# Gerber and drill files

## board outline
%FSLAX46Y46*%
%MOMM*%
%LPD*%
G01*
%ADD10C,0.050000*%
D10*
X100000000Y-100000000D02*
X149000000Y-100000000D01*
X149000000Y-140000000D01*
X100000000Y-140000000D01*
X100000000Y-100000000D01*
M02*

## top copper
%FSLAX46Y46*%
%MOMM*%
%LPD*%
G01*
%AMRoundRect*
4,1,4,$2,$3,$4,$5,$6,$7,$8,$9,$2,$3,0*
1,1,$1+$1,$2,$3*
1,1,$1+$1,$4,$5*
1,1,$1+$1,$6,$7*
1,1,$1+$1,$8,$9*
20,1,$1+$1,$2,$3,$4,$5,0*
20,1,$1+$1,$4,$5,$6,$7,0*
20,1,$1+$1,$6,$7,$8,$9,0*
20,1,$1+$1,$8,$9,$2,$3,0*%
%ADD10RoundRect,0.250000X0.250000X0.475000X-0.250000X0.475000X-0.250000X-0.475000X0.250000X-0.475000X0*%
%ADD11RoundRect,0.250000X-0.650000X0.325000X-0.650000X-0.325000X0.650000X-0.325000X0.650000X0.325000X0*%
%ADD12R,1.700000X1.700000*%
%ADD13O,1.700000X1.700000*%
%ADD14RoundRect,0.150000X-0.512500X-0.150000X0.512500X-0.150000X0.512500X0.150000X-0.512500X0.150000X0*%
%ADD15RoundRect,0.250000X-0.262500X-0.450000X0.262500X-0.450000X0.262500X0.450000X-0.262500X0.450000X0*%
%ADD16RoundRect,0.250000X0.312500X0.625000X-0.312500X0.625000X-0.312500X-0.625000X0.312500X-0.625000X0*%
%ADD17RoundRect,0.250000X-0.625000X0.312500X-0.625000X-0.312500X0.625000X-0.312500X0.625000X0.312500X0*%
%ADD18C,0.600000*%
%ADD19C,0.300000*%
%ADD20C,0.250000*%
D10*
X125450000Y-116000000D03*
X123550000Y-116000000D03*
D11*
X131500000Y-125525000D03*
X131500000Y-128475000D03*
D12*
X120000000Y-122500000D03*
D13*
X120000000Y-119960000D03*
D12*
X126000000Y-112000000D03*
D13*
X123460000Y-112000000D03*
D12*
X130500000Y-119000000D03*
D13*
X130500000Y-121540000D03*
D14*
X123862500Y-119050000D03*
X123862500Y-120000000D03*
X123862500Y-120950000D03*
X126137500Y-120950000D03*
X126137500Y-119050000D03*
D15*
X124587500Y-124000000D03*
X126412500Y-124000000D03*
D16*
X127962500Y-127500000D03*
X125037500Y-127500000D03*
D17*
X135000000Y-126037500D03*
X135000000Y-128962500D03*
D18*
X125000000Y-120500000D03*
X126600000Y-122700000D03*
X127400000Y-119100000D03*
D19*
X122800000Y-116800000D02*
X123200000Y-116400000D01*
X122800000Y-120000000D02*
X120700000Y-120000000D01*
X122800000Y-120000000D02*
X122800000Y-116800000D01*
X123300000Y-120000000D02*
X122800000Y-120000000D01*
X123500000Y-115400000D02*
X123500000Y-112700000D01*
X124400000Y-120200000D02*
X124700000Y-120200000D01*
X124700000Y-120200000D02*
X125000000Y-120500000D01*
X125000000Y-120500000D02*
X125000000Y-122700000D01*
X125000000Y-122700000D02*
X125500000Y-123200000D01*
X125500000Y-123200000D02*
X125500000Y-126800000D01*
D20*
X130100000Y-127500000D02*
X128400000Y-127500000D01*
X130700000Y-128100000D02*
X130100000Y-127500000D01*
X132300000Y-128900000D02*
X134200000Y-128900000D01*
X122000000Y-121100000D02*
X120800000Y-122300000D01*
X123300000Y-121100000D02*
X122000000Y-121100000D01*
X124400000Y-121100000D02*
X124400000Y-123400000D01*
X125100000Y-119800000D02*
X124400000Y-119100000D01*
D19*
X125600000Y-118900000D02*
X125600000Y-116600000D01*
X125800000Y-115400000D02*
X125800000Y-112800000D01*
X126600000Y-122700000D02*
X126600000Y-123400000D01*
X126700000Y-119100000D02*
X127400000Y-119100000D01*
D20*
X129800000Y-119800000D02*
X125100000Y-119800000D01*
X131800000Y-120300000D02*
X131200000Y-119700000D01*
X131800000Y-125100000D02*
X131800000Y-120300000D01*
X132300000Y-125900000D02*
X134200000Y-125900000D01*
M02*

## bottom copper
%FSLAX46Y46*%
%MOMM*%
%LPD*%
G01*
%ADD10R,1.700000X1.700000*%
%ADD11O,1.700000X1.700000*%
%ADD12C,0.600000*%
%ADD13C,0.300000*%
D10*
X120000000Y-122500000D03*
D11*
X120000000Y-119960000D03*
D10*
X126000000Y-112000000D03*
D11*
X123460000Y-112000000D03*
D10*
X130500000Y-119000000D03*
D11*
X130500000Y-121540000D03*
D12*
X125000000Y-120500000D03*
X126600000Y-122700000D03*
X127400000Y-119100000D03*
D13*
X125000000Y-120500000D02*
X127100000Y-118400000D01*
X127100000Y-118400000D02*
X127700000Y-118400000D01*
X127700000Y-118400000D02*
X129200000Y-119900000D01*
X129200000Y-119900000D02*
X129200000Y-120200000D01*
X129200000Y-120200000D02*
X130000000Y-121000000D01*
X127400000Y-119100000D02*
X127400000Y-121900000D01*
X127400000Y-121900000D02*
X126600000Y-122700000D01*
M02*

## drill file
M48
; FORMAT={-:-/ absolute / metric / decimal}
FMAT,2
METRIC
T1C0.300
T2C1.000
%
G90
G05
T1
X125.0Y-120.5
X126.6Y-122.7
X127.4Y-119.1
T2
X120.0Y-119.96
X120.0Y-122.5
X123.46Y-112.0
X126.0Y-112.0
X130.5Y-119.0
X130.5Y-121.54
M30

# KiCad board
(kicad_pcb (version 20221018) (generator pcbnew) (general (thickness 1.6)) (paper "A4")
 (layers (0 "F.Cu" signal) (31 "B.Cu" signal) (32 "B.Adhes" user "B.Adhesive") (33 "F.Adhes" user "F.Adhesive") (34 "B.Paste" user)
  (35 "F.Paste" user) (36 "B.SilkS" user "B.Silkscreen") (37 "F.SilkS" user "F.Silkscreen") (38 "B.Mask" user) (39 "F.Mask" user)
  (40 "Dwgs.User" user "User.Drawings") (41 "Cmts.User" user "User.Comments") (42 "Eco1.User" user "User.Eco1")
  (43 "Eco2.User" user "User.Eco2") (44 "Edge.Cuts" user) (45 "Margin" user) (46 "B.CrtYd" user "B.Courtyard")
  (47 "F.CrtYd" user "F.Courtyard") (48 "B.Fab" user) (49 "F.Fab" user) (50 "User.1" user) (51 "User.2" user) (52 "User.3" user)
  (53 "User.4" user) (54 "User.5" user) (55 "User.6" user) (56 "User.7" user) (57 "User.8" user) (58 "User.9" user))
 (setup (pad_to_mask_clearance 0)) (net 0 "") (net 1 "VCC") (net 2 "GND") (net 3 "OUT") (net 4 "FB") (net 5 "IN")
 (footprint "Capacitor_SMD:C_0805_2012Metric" (layer "F.Cu") (at 124.5 116 180)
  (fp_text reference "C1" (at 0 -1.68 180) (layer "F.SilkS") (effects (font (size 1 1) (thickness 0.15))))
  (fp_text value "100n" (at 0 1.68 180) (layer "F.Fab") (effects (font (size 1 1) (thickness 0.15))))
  (pad "1" smd roundrect (at -0.95 0 180) (size 1 1.45) (layers "F.Cu" "F.Paste" "F.Mask") (roundrect_rratio 0.25) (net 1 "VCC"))
  (pad "2" smd roundrect (at 0.95 0 180) (size 1 1.45) (layers "F.Cu" "F.Paste" "F.Mask") (roundrect_rratio 0.25) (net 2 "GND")))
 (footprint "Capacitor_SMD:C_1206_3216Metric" (layer "F.Cu") (at 131.5 127 -90)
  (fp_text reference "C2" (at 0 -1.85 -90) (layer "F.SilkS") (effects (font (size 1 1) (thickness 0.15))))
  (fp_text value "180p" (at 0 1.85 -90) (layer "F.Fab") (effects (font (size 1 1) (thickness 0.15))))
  (pad "1" smd roundrect (at -1.475 0 270) (size 1.15 1.8) (layers "F.Cu" "F.Paste" "F.Mask") (roundrect_rratio 0.217391) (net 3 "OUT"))
  (pad "2" smd roundrect (at 1.475 0 270) (size 1.15 1.8) (layers "F.Cu" "F.Paste" "F.Mask") (roundrect_rratio 0.217391) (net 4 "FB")))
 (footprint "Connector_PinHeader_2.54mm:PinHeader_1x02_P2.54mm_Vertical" (layer "F.Cu") (at 120 122.5 180)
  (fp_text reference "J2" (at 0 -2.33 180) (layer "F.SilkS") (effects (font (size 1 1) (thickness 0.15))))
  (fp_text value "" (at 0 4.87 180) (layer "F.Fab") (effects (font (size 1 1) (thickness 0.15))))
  (pad "1" thru_hole rect (at 0 0 180) (size 1.7 1.7) (drill 1) (layers "*.Cu" "*.Mask") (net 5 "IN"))
  (pad "2" thru_hole oval (at 0 2.54 180) (size 1.7 1.7) (drill 1) (layers "*.Cu" "*.Mask") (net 2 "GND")))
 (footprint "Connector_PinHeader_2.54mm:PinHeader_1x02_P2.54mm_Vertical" (layer "F.Cu") (at 126 112 -90)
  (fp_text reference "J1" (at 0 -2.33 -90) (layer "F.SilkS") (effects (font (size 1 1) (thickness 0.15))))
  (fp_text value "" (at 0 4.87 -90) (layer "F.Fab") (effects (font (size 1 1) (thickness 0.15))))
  (pad "1" thru_hole rect (at 0 0 270) (size 1.7 1.7) (drill 1) (layers "*.Cu" "*.Mask") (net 1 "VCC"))
  (pad "2" thru_hole oval (at 0 2.54 270) (size 1.7 1.7) (drill 1) (layers "*.Cu" "*.Mask") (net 2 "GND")))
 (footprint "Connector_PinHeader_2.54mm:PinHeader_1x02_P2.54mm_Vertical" (layer "F.Cu") (at 130.5 119)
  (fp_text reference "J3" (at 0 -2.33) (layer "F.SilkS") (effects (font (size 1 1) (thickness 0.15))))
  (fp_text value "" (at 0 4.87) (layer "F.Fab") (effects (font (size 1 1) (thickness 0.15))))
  (pad "1" thru_hole rect (at 0 0) (size 1.7 1.7) (drill 1) (layers "*.Cu" "*.Mask") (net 3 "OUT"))
  (pad "2" thru_hole oval (at 0 2.54) (size 1.7 1.7) (drill 1) (layers "*.Cu" "*.Mask") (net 2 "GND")))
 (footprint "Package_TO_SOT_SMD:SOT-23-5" (layer "F.Cu") (at 125 120)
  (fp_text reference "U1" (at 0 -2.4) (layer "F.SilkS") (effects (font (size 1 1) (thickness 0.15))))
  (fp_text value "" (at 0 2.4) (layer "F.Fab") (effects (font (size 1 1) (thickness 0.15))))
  (pad "1" smd roundrect (at -1.1375 -0.95) (size 1.325 0.6) (layers "F.Cu" "F.Paste" "F.Mask") (roundrect_rratio 0.25) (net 3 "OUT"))
  (pad "2" smd roundrect (at -1.1375 0) (size 1.325 0.6) (layers "F.Cu" "F.Paste" "F.Mask") (roundrect_rratio 0.25) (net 2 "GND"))
  (pad "3" smd roundrect (at -1.1375 0.95) (size 1.325 0.6) (layers "F.Cu" "F.Paste" "F.Mask") (roundrect_rratio 0.25) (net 5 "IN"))
  (pad "4" smd roundrect (at 1.1375 0.95) (size 1.325 0.6) (layers "F.Cu" "F.Paste" "F.Mask") (roundrect_rratio 0.25))
  (pad "5" smd roundrect (at 1.1375 -0.95) (size 1.325 0.6) (layers "F.Cu" "F.Paste" "F.Mask") (roundrect_rratio 0.25) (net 1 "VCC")))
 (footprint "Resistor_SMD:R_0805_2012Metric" (layer "F.Cu") (at 125.5 124)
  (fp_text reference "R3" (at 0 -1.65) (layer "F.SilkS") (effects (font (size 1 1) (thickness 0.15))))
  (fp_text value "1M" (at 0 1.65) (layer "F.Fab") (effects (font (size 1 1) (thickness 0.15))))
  (pad "1" smd roundrect (at -0.9125 0) (size 1.025 1.4) (layers "F.Cu" "F.Paste" "F.Mask") (roundrect_rratio 0.243902) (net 5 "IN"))
  (pad "2" smd roundrect (at 0.9125 0) (size 1.025 1.4) (layers "F.Cu" "F.Paste" "F.Mask") (roundrect_rratio 0.243902) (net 1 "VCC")))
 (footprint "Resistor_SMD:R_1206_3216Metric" (layer "F.Cu") (at 126.5 127.5 180)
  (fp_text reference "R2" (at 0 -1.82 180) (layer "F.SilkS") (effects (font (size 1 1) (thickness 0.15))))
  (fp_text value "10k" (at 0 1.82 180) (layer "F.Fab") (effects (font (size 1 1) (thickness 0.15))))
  (pad "1" smd roundrect (at -1.4625 0 180) (size 1.125 1.75) (layers "F.Cu" "F.Paste" "F.Mask") (roundrect_rratio 0.222222) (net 4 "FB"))
  (pad "2" smd roundrect (at 1.4625 0 180) (size 1.125 1.75) (layers "F.Cu" "F.Paste" "F.Mask") (roundrect_rratio 0.222222) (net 2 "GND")))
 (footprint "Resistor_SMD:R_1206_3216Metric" (layer "F.Cu") (at 135 127.5 -90)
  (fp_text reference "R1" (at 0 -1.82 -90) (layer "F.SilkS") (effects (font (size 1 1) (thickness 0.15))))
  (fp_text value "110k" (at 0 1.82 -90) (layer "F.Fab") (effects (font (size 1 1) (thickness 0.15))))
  (pad "1" smd roundrect (at -1.4625 0 270) (size 1.125 1.75) (layers "F.Cu" "F.Paste" "F.Mask") (roundrect_rratio 0.222222) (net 3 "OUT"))
  (pad "2" smd roundrect (at 1.4625 0 270) (size 1.125 1.75) (layers "F.Cu" "F.Paste" "F.Mask") (roundrect_rratio 0.222222) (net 4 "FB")))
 (gr_rect (start 100 100) (end 149 140) (stroke (width 0.05) (type default)) (fill none) (layer "Edge.Cuts"))
 (segment (start 122.8 116.8) (end 123.2 116.4) (width 0.3) (layer "F.Cu") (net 2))
 (segment (start 122.8 120) (end 120.7 120) (width 0.3) (layer "F.Cu") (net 2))
 (segment (start 122.8 120) (end 122.8 116.8) (width 0.3) (layer "F.Cu") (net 2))
 (segment (start 123.3 120) (end 122.8 120) (width 0.3) (layer "F.Cu") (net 2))
 (segment (start 123.5 115.4) (end 123.5 112.7) (width 0.3) (layer "F.Cu") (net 2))
 (segment (start 124.4 120.2) (end 124.7 120.2) (width 0.3) (layer "F.Cu") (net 2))
 (segment (start 124.7 120.2) (end 125 120.5) (width 0.3) (layer "F.Cu") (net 2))
 (segment (start 125 120.5) (end 125 122.7) (width 0.3) (layer "F.Cu") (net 2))
 (segment (start 125 122.7) (end 125.5 123.2) (width 0.3) (layer "F.Cu") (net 2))
 (segment (start 125.5 123.2) (end 125.5 126.8) (width 0.3) (layer "F.Cu") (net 2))
 (segment (start 130.1 127.5) (end 128.4 127.5) (width 0.25) (layer "F.Cu") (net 4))
 (segment (start 130.7 128.1) (end 130.1 127.5) (width 0.25) (layer "F.Cu") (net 4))
 (segment (start 132.3 128.9) (end 134.2 128.9) (width 0.25) (layer "F.Cu") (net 4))
 (via (at 125 120.5) (size 0.6) (drill 0.3) (layers "F.Cu" "B.Cu") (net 2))
 (segment (start 122 121.1) (end 120.8 122.3) (width 0.25) (layer "F.Cu") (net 5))
 (segment (start 123.3 121.1) (end 122 121.1) (width 0.25) (layer "F.Cu") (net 5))
 (segment (start 124.4 121.1) (end 124.4 123.4) (width 0.25) (layer "F.Cu") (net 5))
 (segment (start 125 120.5) (end 127.1 118.4) (width 0.3) (layer "B.Cu") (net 2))
 (segment (start 125.1 119.8) (end 124.4 119.1) (width 0.25) (layer "F.Cu") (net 3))
 (segment (start 125.6 118.9) (end 125.6 116.6) (width 0.3) (layer "F.Cu") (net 1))
 (segment (start 125.8 115.4) (end 125.8 112.8) (width 0.3) (layer "F.Cu") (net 1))
 (segment (start 126.6 122.7) (end 126.6 123.4) (width 0.3) (layer "F.Cu") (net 1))
 (segment (start 126.7 119.1) (end 127.4 119.1) (width 0.3) (layer "F.Cu") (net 1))
 (segment (start 127.1 118.4) (end 127.7 118.4) (width 0.3) (layer "B.Cu") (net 2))
 (segment (start 127.7 118.4) (end 129.2 119.9) (width 0.3) (layer "B.Cu") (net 2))
 (segment (start 129.2 119.9) (end 129.2 120.2) (width 0.3) (layer "B.Cu") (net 2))
 (segment (start 129.2 120.2) (end 130 121) (width 0.3) (layer "B.Cu") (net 2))
 (segment (start 129.8 119.8) (end 125.1 119.8) (width 0.25) (layer "F.Cu") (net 3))
 (segment (start 131.8 120.3) (end 131.2 119.7) (width 0.25) (layer "F.Cu") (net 3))
 (segment (start 131.8 125.1) (end 131.8 120.3) (width 0.25) (layer "F.Cu") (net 3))
 (segment (start 132.3 125.9) (end 134.2 125.9) (width 0.25) (layer "F.Cu") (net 3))
 (via (at 126.6 122.7) (size 0.6) (drill 0.3) (layers "F.Cu" "B.Cu") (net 1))
 (via (at 127.4 119.1) (size 0.6) (drill 0.3) (layers "F.Cu" "B.Cu") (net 1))
 (segment (start 127.4 119.1) (end 127.4 121.9) (width 0.3) (layer "B.Cu") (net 1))
 (segment (start 127.4 121.9) (end 126.6 122.7) (width 0.3) (layer "B.Cu") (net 1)))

